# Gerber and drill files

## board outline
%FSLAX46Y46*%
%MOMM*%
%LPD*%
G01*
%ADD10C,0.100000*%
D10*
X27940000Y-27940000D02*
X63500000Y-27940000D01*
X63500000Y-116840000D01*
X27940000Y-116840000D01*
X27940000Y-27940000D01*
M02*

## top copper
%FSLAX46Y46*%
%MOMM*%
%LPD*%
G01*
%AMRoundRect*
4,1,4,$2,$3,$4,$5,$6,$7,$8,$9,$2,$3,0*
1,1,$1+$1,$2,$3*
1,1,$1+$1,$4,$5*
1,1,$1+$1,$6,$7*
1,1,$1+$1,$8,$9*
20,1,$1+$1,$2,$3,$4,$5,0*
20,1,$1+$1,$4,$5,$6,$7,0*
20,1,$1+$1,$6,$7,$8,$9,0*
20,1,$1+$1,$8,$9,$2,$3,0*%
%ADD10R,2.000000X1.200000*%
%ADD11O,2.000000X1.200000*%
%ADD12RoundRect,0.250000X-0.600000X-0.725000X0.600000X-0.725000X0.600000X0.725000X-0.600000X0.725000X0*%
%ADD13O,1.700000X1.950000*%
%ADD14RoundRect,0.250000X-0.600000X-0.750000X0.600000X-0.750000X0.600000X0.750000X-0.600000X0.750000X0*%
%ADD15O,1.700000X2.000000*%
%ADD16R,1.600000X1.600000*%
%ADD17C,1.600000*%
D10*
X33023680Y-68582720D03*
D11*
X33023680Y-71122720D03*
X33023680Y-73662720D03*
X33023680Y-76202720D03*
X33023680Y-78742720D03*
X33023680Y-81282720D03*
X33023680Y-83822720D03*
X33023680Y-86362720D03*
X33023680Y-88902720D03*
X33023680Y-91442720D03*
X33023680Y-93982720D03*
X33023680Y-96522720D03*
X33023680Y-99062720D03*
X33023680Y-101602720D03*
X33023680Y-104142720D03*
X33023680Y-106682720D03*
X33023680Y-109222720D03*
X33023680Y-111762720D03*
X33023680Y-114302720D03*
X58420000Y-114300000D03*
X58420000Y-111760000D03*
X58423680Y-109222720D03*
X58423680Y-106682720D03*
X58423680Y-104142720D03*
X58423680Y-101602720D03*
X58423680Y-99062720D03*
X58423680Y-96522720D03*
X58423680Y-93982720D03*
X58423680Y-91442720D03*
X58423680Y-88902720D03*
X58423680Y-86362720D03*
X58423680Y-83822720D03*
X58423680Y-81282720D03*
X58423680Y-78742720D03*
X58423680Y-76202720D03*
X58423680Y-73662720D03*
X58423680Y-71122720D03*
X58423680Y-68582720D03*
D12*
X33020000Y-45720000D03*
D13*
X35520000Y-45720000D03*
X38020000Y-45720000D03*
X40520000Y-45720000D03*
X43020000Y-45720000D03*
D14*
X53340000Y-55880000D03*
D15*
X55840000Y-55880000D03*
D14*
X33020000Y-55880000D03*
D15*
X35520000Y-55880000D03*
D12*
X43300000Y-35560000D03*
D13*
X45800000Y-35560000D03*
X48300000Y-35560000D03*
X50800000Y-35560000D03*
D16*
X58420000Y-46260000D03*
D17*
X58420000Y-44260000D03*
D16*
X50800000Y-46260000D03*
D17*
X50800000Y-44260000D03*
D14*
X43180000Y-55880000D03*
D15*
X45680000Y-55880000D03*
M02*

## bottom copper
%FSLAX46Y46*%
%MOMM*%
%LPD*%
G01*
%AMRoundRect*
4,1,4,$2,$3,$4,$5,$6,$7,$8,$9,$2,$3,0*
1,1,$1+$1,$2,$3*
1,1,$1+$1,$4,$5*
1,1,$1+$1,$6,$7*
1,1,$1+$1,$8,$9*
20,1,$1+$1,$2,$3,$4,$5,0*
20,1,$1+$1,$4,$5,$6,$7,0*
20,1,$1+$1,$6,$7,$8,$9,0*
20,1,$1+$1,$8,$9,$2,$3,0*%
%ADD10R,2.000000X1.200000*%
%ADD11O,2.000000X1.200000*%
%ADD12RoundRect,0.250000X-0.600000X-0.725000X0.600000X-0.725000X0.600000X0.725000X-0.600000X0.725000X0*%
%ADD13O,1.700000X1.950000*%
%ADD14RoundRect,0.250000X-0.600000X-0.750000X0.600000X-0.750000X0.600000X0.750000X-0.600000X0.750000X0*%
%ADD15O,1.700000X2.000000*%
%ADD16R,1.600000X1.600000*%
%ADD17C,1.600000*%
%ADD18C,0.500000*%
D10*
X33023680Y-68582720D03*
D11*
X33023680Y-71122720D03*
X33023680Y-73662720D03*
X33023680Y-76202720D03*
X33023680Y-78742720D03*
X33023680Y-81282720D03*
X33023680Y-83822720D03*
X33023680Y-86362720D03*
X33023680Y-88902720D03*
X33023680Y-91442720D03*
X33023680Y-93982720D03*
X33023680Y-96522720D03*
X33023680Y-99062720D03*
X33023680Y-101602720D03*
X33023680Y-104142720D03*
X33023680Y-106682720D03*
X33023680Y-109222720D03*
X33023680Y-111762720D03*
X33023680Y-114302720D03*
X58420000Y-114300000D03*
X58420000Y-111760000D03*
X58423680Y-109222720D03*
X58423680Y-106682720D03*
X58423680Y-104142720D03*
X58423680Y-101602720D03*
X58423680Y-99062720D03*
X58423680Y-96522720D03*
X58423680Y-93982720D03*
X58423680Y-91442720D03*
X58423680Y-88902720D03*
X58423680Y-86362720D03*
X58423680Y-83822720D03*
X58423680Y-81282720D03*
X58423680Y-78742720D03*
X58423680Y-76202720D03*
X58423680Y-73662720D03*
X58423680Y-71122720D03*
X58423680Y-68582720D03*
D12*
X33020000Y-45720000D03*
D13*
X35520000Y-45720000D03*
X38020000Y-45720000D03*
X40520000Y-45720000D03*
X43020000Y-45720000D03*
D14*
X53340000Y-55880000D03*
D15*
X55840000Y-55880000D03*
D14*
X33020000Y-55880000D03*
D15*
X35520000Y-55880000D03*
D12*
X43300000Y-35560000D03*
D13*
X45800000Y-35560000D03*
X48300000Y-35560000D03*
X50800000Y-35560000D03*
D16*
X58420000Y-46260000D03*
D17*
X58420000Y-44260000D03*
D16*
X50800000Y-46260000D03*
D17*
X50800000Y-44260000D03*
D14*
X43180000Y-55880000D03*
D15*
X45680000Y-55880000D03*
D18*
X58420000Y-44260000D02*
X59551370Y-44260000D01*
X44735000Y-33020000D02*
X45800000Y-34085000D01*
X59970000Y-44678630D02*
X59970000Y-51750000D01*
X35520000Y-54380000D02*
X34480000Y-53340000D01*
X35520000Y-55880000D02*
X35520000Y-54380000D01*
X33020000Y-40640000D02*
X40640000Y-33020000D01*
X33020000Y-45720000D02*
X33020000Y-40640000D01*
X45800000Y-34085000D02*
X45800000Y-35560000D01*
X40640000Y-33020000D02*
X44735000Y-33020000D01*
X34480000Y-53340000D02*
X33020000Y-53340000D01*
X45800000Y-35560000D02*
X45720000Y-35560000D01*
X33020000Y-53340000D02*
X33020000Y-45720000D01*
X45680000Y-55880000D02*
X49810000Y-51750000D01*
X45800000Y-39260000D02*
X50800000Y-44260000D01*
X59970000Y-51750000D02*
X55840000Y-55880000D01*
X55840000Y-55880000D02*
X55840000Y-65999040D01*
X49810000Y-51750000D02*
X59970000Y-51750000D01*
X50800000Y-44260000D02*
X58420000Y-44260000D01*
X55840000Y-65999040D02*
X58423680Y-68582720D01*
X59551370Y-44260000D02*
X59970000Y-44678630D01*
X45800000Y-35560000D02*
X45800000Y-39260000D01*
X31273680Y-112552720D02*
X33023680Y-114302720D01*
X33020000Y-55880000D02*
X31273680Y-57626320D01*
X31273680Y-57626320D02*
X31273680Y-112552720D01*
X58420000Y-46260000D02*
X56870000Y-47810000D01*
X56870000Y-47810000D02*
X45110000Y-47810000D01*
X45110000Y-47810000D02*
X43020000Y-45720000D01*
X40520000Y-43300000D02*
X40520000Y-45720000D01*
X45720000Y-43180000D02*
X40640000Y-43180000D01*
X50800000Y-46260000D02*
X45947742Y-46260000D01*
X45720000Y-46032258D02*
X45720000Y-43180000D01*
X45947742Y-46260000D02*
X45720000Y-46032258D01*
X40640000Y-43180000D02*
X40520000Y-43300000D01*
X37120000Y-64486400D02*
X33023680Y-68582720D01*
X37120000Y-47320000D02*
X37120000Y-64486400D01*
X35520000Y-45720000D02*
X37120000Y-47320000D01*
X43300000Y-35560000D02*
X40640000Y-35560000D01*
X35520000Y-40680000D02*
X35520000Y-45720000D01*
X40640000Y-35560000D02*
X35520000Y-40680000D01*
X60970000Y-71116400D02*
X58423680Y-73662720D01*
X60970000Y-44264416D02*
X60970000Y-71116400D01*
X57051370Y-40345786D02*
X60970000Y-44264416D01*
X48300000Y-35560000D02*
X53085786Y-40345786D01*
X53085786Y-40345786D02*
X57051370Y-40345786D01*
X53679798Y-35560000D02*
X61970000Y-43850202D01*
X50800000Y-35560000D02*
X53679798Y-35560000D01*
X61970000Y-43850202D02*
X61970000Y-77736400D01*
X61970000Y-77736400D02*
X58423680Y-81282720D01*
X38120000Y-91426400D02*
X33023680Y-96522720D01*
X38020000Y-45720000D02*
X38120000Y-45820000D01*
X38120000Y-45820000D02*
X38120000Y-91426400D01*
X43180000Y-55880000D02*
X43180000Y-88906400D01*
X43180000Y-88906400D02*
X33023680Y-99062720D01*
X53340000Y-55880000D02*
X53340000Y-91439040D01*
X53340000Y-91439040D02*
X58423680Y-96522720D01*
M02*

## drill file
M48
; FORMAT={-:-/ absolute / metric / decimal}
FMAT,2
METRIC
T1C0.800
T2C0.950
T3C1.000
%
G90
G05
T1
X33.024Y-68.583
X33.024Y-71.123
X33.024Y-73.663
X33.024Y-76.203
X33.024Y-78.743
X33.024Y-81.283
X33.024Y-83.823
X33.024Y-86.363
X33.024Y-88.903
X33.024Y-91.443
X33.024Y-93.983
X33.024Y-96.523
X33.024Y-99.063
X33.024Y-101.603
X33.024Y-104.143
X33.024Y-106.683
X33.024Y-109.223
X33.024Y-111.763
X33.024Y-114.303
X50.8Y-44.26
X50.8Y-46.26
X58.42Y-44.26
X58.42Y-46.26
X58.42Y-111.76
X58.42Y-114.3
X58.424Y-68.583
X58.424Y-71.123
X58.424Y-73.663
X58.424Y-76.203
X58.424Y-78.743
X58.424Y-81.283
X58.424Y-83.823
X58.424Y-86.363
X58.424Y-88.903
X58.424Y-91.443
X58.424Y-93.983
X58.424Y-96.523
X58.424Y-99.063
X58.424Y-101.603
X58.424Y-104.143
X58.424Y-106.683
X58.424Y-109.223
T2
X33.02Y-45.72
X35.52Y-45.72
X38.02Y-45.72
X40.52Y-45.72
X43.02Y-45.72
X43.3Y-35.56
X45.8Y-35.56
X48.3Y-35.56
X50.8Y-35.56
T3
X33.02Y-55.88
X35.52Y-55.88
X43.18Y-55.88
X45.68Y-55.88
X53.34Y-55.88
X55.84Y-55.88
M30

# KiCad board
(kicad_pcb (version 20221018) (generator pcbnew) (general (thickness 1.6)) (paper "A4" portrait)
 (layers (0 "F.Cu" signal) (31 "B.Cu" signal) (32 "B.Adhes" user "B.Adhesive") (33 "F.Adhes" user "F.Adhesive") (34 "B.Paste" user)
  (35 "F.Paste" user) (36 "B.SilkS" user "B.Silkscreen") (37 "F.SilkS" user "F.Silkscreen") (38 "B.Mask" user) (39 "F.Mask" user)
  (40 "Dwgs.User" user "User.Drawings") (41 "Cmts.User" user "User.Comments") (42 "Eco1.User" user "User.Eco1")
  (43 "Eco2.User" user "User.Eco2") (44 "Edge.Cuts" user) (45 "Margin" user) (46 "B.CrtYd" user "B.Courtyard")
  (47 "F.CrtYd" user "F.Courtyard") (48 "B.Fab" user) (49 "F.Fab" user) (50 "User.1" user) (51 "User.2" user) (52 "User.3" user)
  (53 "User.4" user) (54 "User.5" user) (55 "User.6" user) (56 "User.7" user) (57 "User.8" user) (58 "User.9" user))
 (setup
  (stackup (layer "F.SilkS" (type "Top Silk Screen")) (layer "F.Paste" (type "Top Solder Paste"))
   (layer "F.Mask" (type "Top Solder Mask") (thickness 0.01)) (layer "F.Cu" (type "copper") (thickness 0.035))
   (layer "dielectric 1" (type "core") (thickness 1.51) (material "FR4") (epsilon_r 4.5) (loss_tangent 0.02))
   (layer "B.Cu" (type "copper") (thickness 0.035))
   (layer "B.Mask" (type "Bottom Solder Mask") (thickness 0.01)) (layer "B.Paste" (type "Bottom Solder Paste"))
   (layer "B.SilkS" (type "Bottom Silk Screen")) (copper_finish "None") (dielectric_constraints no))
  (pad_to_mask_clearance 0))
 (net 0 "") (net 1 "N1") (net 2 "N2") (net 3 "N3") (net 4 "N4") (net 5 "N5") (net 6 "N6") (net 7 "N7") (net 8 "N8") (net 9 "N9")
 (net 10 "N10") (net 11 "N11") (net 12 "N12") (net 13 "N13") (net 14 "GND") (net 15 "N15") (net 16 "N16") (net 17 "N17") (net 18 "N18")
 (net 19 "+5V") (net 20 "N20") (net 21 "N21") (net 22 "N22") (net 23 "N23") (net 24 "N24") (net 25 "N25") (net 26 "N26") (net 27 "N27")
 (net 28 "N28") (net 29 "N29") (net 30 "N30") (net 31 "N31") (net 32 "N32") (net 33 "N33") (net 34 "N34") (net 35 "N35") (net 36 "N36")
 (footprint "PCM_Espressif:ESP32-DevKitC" (layer "F.Cu") (at 33.02368 68.58272)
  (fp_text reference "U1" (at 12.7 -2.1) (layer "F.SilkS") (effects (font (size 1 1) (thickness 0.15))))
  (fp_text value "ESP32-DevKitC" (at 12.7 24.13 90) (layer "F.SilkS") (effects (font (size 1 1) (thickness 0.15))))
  (pad "1" thru_hole rect (at 0 0 270) (size 1.2 2) (drill 0.8) (layers "*.Cu" "*.Mask") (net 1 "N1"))
  (pad "2" thru_hole oval (at 0 2.54 270) (size 1.2 2) (drill 0.8) (layers "*.Cu" "*.Mask") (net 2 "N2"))
  (pad "3" thru_hole oval (at 0 5.08 270) (size 1.2 2) (drill 0.8) (layers "*.Cu" "*.Mask") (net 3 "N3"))
  (pad "4" thru_hole oval (at 0 7.62 270) (size 1.2 2) (drill 0.8) (layers "*.Cu" "*.Mask") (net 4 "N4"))
  (pad "5" thru_hole oval (at 0 10.16 270) (size 1.2 2) (drill 0.8) (layers "*.Cu" "*.Mask") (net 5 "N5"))
  (pad "6" thru_hole oval (at 0 12.7 270) (size 1.2 2) (drill 0.8) (layers "*.Cu" "*.Mask") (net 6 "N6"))
  (pad "7" thru_hole oval (at 0 15.24 270) (size 1.2 2) (drill 0.8) (layers "*.Cu" "*.Mask") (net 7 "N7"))
  (pad "8" thru_hole oval (at 0 17.78 270) (size 1.2 2) (drill 0.8) (layers "*.Cu" "*.Mask") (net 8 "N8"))
  (pad "9" thru_hole oval (at 0 20.32 270) (size 1.2 2) (drill 0.8) (layers "*.Cu" "*.Mask") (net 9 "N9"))
  (pad "10" thru_hole oval (at 0 22.86 270) (size 1.2 2) (drill 0.8) (layers "*.Cu" "*.Mask") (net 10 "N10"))
  (pad "11" thru_hole oval (at 0 25.4 270) (size 1.2 2) (drill 0.8) (layers "*.Cu" "*.Mask") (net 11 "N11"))
  (pad "12" thru_hole oval (at 0 27.94 270) (size 1.2 2) (drill 0.8) (layers "*.Cu" "*.Mask") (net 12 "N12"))
  (pad "13" thru_hole oval (at 0 30.48 270) (size 1.2 2) (drill 0.8) (layers "*.Cu" "*.Mask") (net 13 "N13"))
  (pad "14" thru_hole oval (at 0 33.02 270) (size 1.2 2) (drill 0.8) (layers "*.Cu" "*.Mask") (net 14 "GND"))
  (pad "15" thru_hole oval (at 0 35.56 270) (size 1.2 2) (drill 0.8) (layers "*.Cu" "*.Mask") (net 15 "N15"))
  (pad "16" thru_hole oval (at 0 38.1 270) (size 1.2 2) (drill 0.8) (layers "*.Cu" "*.Mask") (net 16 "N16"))
  (pad "17" thru_hole oval (at 0 40.64 270) (size 1.2 2) (drill 0.8) (layers "*.Cu" "*.Mask") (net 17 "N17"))
  (pad "18" thru_hole oval (at 0 43.18 270) (size 1.2 2) (drill 0.8) (layers "*.Cu" "*.Mask") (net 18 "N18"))
  (pad "19" thru_hole oval (at 0 45.72 270) (size 1.2 2) (drill 0.8) (layers "*.Cu" "*.Mask") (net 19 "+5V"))
  (pad "20" thru_hole oval (at 25.39632 45.71728 270) (size 1.2 2) (drill 0.8) (layers "*.Cu" "*.Mask") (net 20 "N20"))
  (pad "21" thru_hole oval (at 25.39632 43.17728 270) (size 1.2 2) (drill 0.8) (layers "*.Cu" "*.Mask") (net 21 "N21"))
  (pad "22" thru_hole oval (at 25.4 40.64 270) (size 1.2 2) (drill 0.8) (layers "*.Cu" "*.Mask") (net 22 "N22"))
  (pad "23" thru_hole oval (at 25.4 38.1 270) (size 1.2 2) (drill 0.8) (layers "*.Cu" "*.Mask") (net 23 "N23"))
  (pad "24" thru_hole oval (at 25.4 35.56 270) (size 1.2 2) (drill 0.8) (layers "*.Cu" "*.Mask") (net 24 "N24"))
  (pad "25" thru_hole oval (at 25.4 33.02 270) (size 1.2 2) (drill 0.8) (layers "*.Cu" "*.Mask") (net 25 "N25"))
  (pad "26" thru_hole oval (at 25.4 30.48 270) (size 1.2 2) (drill 0.8) (layers "*.Cu" "*.Mask") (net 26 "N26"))
  (pad "27" thru_hole oval (at 25.4 27.94 270) (size 1.2 2) (drill 0.8) (layers "*.Cu" "*.Mask") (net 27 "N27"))
  (pad "28" thru_hole oval (at 25.4 25.4 270) (size 1.2 2) (drill 0.8) (layers "*.Cu" "*.Mask") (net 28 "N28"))
  (pad "29" thru_hole oval (at 25.4 22.86 270) (size 1.2 2) (drill 0.8) (layers "*.Cu" "*.Mask") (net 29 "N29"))
  (pad "30" thru_hole oval (at 25.4 20.32 270) (size 1.2 2) (drill 0.8) (layers "*.Cu" "*.Mask") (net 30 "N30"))
  (pad "31" thru_hole oval (at 25.4 17.78 270) (size 1.2 2) (drill 0.8) (layers "*.Cu" "*.Mask") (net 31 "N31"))
  (pad "32" thru_hole oval (at 25.4 15.24 270) (size 1.2 2) (drill 0.8) (layers "*.Cu" "*.Mask") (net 14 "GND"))
  (pad "33" thru_hole oval (at 25.4 12.7 270) (size 1.2 2) (drill 0.8) (layers "*.Cu" "*.Mask") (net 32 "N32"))
  (pad "34" thru_hole oval (at 25.4 10.16 270) (size 1.2 2) (drill 0.8) (layers "*.Cu" "*.Mask") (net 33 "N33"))
  (pad "35" thru_hole oval (at 25.4 7.62 270) (size 1.2 2) (drill 0.8) (layers "*.Cu" "*.Mask") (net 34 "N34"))
  (pad "36" thru_hole oval (at 25.4 5.08 270) (size 1.2 2) (drill 0.8) (layers "*.Cu" "*.Mask") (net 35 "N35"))
  (pad "37" thru_hole oval (at 25.4 2.54 270) (size 1.2 2) (drill 0.8) (layers "*.Cu" "*.Mask") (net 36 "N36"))
  (pad "38" thru_hole oval (at 25.4 0 270) (size 1.2 2) (drill 0.8) (layers "*.Cu" "*.Mask") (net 14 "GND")))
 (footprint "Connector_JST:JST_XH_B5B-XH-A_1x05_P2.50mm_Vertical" (layer "F.Cu") (at 33.02 45.72)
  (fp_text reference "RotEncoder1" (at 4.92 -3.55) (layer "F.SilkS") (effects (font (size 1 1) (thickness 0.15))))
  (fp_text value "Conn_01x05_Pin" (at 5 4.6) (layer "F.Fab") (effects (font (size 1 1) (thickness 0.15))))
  (pad "1" thru_hole roundrect (at 0 0) (size 1.7 1.95) (drill 0.95) (layers "*.Cu" "*.Mask") (roundrect_rratio 0.1470588235) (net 14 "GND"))
  (pad "2" thru_hole oval (at 2.5 0) (size 1.7 1.95) (drill 0.95) (layers "*.Cu" "*.Mask") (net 1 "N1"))
  (pad "3" thru_hole oval (at 5 0) (size 1.7 1.95) (drill 0.95) (layers "*.Cu" "*.Mask") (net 12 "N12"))
  (pad "4" thru_hole oval (at 7.5 0) (size 1.7 1.95) (drill 0.95) (layers "*.Cu" "*.Mask") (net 30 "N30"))
  (pad "5" thru_hole oval (at 10 0) (size 1.7 1.95) (drill 0.95) (layers "*.Cu" "*.Mask") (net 31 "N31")))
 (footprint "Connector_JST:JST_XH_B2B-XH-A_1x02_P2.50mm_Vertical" (layer "F.Cu") (at 53.34 55.88)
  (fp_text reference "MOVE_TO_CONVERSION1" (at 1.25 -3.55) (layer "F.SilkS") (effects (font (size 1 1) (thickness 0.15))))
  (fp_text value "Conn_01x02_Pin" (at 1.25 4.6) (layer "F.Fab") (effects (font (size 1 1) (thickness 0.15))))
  (pad "1" thru_hole roundrect (at 0 0) (size 1.7 2) (drill 1) (layers "*.Cu" "*.Mask") (roundrect_rratio 0.1470588235) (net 27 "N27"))
  (pad "2" thru_hole oval (at 2.5 0) (size 1.7 2) (drill 1) (layers "*.Cu" "*.Mask") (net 14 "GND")))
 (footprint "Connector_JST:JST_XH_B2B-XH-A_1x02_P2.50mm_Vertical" (layer "F.Cu") (at 33.02 55.88)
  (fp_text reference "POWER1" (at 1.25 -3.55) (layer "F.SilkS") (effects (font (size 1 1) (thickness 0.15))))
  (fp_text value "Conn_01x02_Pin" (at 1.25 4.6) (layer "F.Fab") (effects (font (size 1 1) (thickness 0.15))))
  (pad "1" thru_hole roundrect (at 0 0) (size 1.7 2) (drill 1) (layers "*.Cu" "*.Mask") (roundrect_rratio 0.1470588235) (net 19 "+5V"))
  (pad "2" thru_hole oval (at 2.5 0) (size 1.7 2) (drill 1) (layers "*.Cu" "*.Mask") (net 14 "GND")))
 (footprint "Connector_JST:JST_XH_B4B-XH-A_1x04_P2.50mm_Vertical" (layer "F.Cu") (at 43.3 35.56)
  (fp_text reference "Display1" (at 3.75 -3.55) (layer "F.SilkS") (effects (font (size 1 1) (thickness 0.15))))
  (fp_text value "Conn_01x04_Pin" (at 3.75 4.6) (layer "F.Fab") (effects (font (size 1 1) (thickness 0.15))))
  (pad "1" thru_hole roundrect (at 0 0) (size 1.7 1.95) (drill 0.95) (layers "*.Cu" "*.Mask") (roundrect_rratio 0.1470588235) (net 1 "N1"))
  (pad "2" thru_hole oval (at 2.5 0) (size 1.7 1.95) (drill 0.95) (layers "*.Cu" "*.Mask") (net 14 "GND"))
  (pad "3" thru_hole oval (at 5 0) (size 1.7 1.95) (drill 0.95) (layers "*.Cu" "*.Mask") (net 35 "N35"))
  (pad "4" thru_hole oval (at 7.5 0) (size 1.7 1.95) (drill 0.95) (layers "*.Cu" "*.Mask") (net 32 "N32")))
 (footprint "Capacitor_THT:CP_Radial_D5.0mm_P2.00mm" (layer "F.Cu") (at 58.42 46.26 90)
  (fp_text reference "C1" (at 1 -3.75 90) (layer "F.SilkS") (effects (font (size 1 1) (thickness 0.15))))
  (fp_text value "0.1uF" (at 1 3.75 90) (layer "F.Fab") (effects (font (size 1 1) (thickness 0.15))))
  (pad "1" thru_hole rect (at 0 0 90) (size 1.6 1.6) (drill 0.8) (layers "*.Cu" "*.Mask") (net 31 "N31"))
  (pad "2" thru_hole circle (at 2 0 90) (size 1.6 1.6) (drill 0.8) (layers "*.Cu" "*.Mask") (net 14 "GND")))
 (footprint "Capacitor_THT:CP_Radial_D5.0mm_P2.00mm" (layer "F.Cu") (at 50.8 46.26 90)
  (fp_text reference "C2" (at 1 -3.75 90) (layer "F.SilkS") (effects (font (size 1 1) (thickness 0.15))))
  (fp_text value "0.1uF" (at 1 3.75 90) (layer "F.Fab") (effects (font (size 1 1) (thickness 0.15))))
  (pad "1" thru_hole rect (at 0 0 90) (size 1.6 1.6) (drill 0.8) (layers "*.Cu" "*.Mask") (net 30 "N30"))
  (pad "2" thru_hole circle (at 2 0 90) (size 1.6 1.6) (drill 0.8) (layers "*.Cu" "*.Mask") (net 14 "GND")))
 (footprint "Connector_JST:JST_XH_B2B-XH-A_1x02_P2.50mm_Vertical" (layer "F.Cu") (at 43.18 55.88)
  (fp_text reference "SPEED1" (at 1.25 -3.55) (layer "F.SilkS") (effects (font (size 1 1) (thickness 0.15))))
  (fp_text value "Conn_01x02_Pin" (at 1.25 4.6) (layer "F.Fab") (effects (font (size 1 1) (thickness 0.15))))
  (pad "1" thru_hole roundrect (at 0 0) (size 1.7 2) (drill 1) (layers "*.Cu" "*.Mask") (roundrect_rratio 0.1470588235) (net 13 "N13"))
  (pad "2" thru_hole oval (at 2.5 0) (size 1.7 2) (drill 1) (layers "*.Cu" "*.Mask") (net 14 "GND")))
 (gr_rect (start 27.94 27.94) (end 63.5 116.84) (stroke (width 0.1) (type default)) (fill none) (layer "Edge.Cuts"))
 (segment (start 58.42 44.26) (end 59.55137 44.26) (width 0.5) (layer "B.Cu") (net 14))
 (segment (start 44.735 33.02) (end 45.8 34.085) (width 0.5) (layer "B.Cu") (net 14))
 (segment (start 59.97 44.67863) (end 59.97 51.75) (width 0.5) (layer "B.Cu") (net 14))
 (segment (start 35.52 54.38) (end 34.48 53.34) (width 0.5) (layer "B.Cu") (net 14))
 (segment (start 35.52 55.88) (end 35.52 54.38) (width 0.5) (layer "B.Cu") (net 14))
 (segment (start 33.02 40.64) (end 40.64 33.02) (width 0.5) (layer "B.Cu") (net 14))
 (segment (start 33.02 45.72) (end 33.02 40.64) (width 0.5) (layer "B.Cu") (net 14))
 (segment (start 45.8 34.085) (end 45.8 35.56) (width 0.5) (layer "B.Cu") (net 14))
 (segment (start 40.64 33.02) (end 44.735 33.02) (width 0.5) (layer "B.Cu") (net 14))
 (segment (start 34.48 53.34) (end 33.02 53.34) (width 0.5) (layer "B.Cu") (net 14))
 (segment (start 45.8 35.56) (end 45.72 35.56) (width 0.5) (layer "B.Cu") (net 14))
 (segment (start 33.02 53.34) (end 33.02 45.72) (width 0.5) (layer "B.Cu") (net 14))
 (segment (start 45.68 55.88) (end 49.81 51.75) (width 0.5) (layer "B.Cu") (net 14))
 (segment (start 45.8 39.26) (end 50.8 44.26) (width 0.5) (layer "B.Cu") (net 14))
 (segment (start 59.97 51.75) (end 55.84 55.88) (width 0.5) (layer "B.Cu") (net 14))
 (segment (start 55.84 55.88) (end 55.84 65.99904) (width 0.5) (layer "B.Cu") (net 14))
 (segment (start 49.81 51.75) (end 59.97 51.75) (width 0.5) (layer "B.Cu") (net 14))
 (segment (start 50.8 44.26) (end 58.42 44.26) (width 0.5) (layer "B.Cu") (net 14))
 (segment (start 55.84 65.99904) (end 58.42368 68.58272) (width 0.5) (layer "B.Cu") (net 14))
 (segment (start 59.55137 44.26) (end 59.97 44.67863) (width 0.5) (layer "B.Cu") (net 14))
 (segment (start 45.8 35.56) (end 45.8 39.26) (width 0.5) (layer "B.Cu") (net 14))
 (segment (start 31.27368 112.55272) (end 33.02368 114.30272) (width 0.5) (layer "B.Cu") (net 19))
 (segment (start 33.02 55.88) (end 31.27368 57.62632) (width 0.5) (layer "B.Cu") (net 19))
 (segment (start 31.27368 57.62632) (end 31.27368 112.55272) (width 0.5) (layer "B.Cu") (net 19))
 (segment (start 58.42 46.26) (end 56.87 47.81) (width 0.5) (layer "B.Cu") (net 31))
 (segment (start 56.87 47.81) (end 45.11 47.81) (width 0.5) (layer "B.Cu") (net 31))
 (segment (start 45.11 47.81) (end 43.02 45.72) (width 0.5) (layer "B.Cu") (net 31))
 (segment (start 40.52 43.3) (end 40.52 45.72) (width 0.5) (layer "B.Cu") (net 30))
 (segment (start 45.72 43.18) (end 40.64 43.18) (width 0.5) (layer "B.Cu") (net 30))
 (segment (start 50.8 46.26) (end 45.947742 46.26) (width 0.5) (layer "B.Cu") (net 30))
 (segment (start 45.72 46.032258) (end 45.72 43.18) (width 0.5) (layer "B.Cu") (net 30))
 (segment (start 45.947742 46.26) (end 45.72 46.032258) (width 0.5) (layer "B.Cu") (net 30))
 (segment (start 40.64 43.18) (end 40.52 43.3) (width 0.5) (layer "B.Cu") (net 30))
 (segment (start 37.12 64.4864) (end 33.02368 68.58272) (width 0.5) (layer "B.Cu") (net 1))
 (segment (start 37.12 47.32) (end 37.12 64.4864) (width 0.5) (layer "B.Cu") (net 1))
 (segment (start 35.52 45.72) (end 37.12 47.32) (width 0.5) (layer "B.Cu") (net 1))
 (segment (start 43.3 35.56) (end 40.64 35.56) (width 0.5) (layer "B.Cu") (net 1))
 (segment (start 35.52 40.68) (end 35.52 45.72) (width 0.5) (layer "B.Cu") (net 1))
 (segment (start 40.64 35.56) (end 35.52 40.68) (width 0.5) (layer "B.Cu") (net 1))
 (segment (start 60.97 71.1164) (end 58.42368 73.66272) (width 0.5) (layer "B.Cu") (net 35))
 (segment (start 60.97 44.264416) (end 60.97 71.1164) (width 0.5) (layer "B.Cu") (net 35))
 (segment (start 57.05137 40.345786) (end 60.97 44.264416) (width 0.5) (layer "B.Cu") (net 35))
 (segment (start 48.3 35.56) (end 53.085786 40.345786) (width 0.5) (layer "B.Cu") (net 35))
 (segment (start 53.085786 40.345786) (end 57.05137 40.345786) (width 0.5) (layer "B.Cu") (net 35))
 (segment (start 53.679798 35.56) (end 61.97 43.850202) (width 0.5) (layer "B.Cu") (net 32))
 (segment (start 50.8 35.56) (end 53.679798 35.56) (width 0.5) (layer "B.Cu") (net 32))
 (segment (start 61.97 43.850202) (end 61.97 77.7364) (width 0.5) (layer "B.Cu") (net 32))
 (segment (start 61.97 77.7364) (end 58.42368 81.28272) (width 0.5) (layer "B.Cu") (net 32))
 (segment (start 38.12 91.4264) (end 33.02368 96.52272) (width 0.5) (layer "B.Cu") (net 12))
 (segment (start 38.02 45.72) (end 38.12 45.82) (width 0.5) (layer "B.Cu") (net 12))
 (segment (start 38.12 45.82) (end 38.12 91.4264) (width 0.5) (layer "B.Cu") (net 12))
 (segment (start 43.18 55.88) (end 43.18 88.9064) (width 0.5) (layer "B.Cu") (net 13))
 (segment (start 43.18 88.9064) (end 33.02368 99.06272) (width 0.5) (layer "B.Cu") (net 13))
 (segment (start 53.34 55.88) (end 53.34 91.43904) (width 0.5) (layer "B.Cu") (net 27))
 (segment (start 53.34 91.43904) (end 58.42368 96.52272) (width 0.5) (layer "B.Cu") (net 27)))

